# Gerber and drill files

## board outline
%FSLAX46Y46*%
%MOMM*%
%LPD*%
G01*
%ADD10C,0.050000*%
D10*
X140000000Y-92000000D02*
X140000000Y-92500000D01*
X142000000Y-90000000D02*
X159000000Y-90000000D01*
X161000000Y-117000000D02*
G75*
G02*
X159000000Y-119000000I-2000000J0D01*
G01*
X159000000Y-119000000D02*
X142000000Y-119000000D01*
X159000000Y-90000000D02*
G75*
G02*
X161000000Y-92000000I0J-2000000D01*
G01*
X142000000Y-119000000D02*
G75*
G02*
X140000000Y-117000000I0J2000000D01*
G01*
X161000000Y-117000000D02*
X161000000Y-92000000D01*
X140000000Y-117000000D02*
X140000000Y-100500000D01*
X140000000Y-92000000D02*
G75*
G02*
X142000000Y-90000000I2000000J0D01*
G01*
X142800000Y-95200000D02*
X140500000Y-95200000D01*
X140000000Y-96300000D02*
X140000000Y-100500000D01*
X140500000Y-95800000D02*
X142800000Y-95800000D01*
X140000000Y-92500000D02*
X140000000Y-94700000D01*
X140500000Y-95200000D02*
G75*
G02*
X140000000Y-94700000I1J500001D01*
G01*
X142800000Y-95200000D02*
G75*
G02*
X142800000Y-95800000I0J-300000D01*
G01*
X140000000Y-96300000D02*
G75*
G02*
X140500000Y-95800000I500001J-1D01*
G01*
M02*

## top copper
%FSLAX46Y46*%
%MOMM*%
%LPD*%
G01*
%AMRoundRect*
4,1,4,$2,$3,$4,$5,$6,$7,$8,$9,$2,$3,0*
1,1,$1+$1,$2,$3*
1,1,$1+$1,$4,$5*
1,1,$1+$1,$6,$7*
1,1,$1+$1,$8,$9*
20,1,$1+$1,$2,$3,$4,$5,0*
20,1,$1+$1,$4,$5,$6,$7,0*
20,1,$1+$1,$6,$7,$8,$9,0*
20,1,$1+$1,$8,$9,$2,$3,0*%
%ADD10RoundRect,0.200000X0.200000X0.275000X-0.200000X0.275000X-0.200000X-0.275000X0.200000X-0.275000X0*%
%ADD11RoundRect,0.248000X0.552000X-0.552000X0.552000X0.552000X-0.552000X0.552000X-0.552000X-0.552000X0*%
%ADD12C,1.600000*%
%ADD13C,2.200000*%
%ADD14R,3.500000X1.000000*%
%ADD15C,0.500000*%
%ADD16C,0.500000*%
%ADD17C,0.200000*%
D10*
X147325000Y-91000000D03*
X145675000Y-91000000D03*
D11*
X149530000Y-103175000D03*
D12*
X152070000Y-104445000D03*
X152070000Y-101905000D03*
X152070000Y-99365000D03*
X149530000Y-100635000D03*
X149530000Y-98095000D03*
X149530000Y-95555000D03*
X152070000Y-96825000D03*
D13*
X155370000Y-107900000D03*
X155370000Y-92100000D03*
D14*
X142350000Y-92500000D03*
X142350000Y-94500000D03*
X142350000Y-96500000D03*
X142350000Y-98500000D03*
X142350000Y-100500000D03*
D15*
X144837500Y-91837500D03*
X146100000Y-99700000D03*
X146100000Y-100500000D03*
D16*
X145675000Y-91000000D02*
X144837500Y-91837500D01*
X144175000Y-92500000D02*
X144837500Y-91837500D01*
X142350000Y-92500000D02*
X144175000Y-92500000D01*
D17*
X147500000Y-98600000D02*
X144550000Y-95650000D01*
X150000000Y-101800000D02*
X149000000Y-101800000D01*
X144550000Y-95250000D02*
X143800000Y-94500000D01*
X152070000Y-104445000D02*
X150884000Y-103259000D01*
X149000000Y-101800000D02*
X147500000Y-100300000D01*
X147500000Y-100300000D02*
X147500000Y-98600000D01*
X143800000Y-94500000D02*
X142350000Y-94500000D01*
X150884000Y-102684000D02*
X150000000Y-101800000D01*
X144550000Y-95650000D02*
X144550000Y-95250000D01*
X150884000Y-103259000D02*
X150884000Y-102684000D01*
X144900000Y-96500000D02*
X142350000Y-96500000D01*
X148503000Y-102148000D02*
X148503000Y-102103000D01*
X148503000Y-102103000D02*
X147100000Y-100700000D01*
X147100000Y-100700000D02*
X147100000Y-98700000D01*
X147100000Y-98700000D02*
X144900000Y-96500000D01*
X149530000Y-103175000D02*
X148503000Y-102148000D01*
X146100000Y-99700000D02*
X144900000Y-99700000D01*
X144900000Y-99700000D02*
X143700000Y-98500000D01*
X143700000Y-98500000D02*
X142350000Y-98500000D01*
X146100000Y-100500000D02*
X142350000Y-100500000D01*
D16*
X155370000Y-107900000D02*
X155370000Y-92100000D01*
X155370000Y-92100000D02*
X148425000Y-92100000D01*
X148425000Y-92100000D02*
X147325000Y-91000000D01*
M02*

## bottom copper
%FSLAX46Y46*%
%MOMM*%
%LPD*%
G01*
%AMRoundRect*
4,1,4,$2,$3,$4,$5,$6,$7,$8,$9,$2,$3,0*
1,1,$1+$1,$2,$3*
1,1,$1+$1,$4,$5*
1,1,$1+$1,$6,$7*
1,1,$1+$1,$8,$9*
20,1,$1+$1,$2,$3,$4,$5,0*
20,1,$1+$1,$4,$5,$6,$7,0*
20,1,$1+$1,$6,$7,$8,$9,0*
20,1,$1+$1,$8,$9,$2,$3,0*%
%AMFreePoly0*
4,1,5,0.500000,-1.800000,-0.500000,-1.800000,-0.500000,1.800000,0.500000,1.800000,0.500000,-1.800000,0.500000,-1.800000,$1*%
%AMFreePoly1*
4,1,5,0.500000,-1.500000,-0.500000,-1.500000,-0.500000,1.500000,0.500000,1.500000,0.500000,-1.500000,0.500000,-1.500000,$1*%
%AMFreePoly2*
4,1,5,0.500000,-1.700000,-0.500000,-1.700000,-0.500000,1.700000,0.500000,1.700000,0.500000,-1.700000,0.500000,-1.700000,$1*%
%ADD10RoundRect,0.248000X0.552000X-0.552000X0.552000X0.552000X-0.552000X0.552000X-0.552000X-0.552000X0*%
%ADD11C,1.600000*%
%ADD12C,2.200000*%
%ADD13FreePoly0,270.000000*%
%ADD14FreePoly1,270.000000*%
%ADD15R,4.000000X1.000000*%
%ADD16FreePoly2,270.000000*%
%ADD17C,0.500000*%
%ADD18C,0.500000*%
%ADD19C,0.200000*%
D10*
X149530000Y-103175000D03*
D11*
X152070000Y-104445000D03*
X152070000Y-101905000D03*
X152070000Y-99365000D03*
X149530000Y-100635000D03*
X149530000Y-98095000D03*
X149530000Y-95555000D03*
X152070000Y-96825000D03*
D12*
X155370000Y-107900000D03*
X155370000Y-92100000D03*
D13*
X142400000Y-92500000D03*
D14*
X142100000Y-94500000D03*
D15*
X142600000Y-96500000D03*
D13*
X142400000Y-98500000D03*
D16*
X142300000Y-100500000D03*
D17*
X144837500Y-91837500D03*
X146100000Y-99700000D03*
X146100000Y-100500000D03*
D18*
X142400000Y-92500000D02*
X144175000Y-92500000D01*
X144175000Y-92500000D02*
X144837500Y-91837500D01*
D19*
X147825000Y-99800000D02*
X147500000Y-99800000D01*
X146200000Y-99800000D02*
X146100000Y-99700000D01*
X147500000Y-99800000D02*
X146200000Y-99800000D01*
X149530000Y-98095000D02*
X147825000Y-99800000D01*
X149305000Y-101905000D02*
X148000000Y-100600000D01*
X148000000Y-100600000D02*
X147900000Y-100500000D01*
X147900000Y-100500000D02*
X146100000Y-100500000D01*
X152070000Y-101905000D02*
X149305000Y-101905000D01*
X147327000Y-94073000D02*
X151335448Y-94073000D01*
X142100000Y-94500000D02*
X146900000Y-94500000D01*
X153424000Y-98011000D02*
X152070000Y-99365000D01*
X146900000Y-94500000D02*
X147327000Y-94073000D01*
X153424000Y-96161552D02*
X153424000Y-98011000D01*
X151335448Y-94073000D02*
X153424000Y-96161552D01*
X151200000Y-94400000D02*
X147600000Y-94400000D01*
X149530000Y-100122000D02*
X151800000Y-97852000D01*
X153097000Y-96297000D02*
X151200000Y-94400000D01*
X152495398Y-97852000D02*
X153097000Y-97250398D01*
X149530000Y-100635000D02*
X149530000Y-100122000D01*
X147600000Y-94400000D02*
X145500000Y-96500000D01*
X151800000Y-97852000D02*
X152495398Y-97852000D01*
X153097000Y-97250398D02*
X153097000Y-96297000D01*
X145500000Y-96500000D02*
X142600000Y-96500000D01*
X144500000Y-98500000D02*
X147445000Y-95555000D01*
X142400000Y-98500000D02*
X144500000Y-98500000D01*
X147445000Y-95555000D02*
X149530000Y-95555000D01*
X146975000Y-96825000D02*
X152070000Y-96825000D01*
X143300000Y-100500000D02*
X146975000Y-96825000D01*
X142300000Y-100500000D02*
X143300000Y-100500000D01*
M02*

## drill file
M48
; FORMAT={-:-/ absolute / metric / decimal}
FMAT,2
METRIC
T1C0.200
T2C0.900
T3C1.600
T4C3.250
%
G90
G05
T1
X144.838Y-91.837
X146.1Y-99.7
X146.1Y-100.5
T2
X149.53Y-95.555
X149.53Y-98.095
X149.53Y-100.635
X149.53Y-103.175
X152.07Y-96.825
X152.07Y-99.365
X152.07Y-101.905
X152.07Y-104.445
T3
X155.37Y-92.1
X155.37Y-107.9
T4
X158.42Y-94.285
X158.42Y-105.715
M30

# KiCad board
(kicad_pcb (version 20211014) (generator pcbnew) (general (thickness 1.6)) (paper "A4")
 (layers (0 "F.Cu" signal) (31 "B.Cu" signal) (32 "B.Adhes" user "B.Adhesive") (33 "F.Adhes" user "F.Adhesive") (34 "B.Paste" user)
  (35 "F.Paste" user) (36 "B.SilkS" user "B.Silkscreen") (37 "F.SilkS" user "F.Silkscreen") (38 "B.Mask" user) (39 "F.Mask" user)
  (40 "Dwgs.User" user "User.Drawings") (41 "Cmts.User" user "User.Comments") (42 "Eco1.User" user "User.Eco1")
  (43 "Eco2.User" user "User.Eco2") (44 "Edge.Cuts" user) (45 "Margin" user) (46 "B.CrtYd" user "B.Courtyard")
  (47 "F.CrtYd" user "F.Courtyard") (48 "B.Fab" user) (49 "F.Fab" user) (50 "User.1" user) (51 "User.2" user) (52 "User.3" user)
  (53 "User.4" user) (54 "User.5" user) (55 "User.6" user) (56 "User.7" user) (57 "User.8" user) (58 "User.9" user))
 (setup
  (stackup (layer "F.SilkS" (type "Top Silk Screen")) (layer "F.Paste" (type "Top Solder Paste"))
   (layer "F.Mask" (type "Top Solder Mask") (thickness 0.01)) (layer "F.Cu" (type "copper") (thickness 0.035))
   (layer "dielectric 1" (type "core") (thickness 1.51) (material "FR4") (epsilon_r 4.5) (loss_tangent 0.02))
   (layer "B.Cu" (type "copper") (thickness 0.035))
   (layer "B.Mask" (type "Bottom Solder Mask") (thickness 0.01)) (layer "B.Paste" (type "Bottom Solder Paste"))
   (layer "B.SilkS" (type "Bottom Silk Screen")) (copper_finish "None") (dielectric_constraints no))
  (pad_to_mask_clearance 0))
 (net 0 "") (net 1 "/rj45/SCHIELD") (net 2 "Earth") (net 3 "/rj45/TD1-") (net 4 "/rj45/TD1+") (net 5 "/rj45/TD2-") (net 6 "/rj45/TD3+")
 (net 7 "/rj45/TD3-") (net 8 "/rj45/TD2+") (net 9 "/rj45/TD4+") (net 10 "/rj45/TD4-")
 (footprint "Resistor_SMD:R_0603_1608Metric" (layer "F.Cu") (at 146.5 91 180)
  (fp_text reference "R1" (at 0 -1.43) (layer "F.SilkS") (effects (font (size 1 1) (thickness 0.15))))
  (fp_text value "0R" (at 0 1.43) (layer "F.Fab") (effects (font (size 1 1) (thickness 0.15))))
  (pad "1" smd roundrect (at -0.825 0 180) (size 0.8 0.95) (layers "F.Cu" "F.Paste" "F.Mask") (roundrect_rratio 0.25)
   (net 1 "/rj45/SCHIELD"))
  (pad "2" smd roundrect (at 0.825 0 180) (size 0.8 0.95) (layers "F.Cu" "F.Paste" "F.Mask") (roundrect_rratio 0.25) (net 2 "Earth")))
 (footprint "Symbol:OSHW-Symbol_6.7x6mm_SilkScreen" (layer "F.Cu") (at 143.5 115)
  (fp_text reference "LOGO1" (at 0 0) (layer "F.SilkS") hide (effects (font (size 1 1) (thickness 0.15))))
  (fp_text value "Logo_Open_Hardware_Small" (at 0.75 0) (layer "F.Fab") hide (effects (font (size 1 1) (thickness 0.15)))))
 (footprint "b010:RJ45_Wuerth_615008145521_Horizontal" (layer "F.Cu") (at 149.53 95.555)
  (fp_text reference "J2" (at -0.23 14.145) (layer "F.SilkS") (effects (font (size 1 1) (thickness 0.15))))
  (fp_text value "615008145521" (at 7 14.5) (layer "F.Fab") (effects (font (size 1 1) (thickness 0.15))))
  (pad "" np_thru_hole circle (at 8.89 10.16 90) (size 3.25 3.25) (drill 3.25) (layers *.Cu *.Mask))
  (pad "" np_thru_hole circle (at 8.89 -1.27 90) (size 3.25 3.25) (drill 3.25) (layers *.Cu *.Mask))
  (pad "1" thru_hole roundrect (at 0 7.62 90) (size 1.6 1.6) (drill 0.9) (layers *.Cu *.Mask) (roundrect_rratio 0.155) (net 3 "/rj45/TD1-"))
  (pad "2" thru_hole circle (at 2.54 8.89 90) (size 1.6 1.6) (drill 0.9) (layers *.Cu *.Mask) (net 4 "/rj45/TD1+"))
  (pad "3" thru_hole circle (at 2.54 6.35 90) (size 1.6 1.6) (drill 0.9) (layers *.Cu *.Mask) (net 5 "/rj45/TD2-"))
  (pad "4" thru_hole circle (at 2.54 3.81 90) (size 1.6 1.6) (drill 0.9) (layers *.Cu *.Mask) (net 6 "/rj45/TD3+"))
  (pad "5" thru_hole circle (at 0 5.08 90) (size 1.6 1.6) (drill 0.9) (layers *.Cu *.Mask) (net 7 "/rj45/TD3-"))
  (pad "6" thru_hole circle (at 0 2.54 90) (size 1.6 1.6) (drill 0.9) (layers *.Cu *.Mask) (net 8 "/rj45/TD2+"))
  (pad "7" thru_hole circle (at 0 0 90) (size 1.6 1.6) (drill 0.9) (layers *.Cu *.Mask) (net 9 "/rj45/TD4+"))
  (pad "8" thru_hole circle (at 2.54 1.27 90) (size 1.6 1.6) (drill 0.9) (layers *.Cu *.Mask) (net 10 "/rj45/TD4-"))
  (pad "SH" thru_hole circle (at 5.84 12.345 90) (size 2.2 2.2) (drill 1.6) (layers *.Cu *.Mask) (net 1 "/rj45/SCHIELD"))
  (pad "SH" thru_hole circle (at 5.84 -3.455 90) (size 2.2 2.2) (drill 1.6) (layers *.Cu *.Mask) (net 1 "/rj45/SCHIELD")))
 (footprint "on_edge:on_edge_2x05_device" (layer "F.Cu") (at 140 96.5 -90)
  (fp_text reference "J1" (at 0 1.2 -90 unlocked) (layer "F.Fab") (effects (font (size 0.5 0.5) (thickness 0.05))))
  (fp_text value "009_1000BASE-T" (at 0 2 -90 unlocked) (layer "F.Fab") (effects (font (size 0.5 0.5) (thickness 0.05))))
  (fp_line (start -1.3 -2.8) (end -1.3 -0.5) (layer "Edge.Cuts") (width 0.05))
  (fp_line (start -0.2 0) (end 4 0) (layer "Edge.Cuts") (width 0.05))
  (fp_line (start -0.7 -0.5) (end -0.7 -2.8) (layer "Edge.Cuts") (width 0.05))
  (fp_line (start -4 0) (end -1.8 0) (layer "Edge.Cuts") (width 0.05))
  (fp_arc (start -1.3 -0.5) (mid -1.446447 -0.146447) (end -1.8 0) (layer "Edge.Cuts") (width 0.05))
  (fp_arc (start -1.3 -2.8) (mid -1 -3.1) (end -0.7 -2.8) (layer "Edge.Cuts") (width 0.05))
  (fp_arc (start -0.2 0) (mid -0.553553 -0.146447) (end -0.7 -0.5) (layer "Edge.Cuts") (width 0.05))
  (pad "1" smd rect (at -4 -2.35 90) (size 1 3.5) (layers "F.Cu" "F.Mask") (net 2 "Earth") (zone_connect 0))
  (pad "2" smd rect (at -2 -2.35 270) (size 1 3.5) (layers "F.Cu" "F.Mask") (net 4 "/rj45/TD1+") (zone_connect 0))
  (pad "3" smd rect (at 0 -2.35 270) (size 1 3.5) (layers "F.Cu" "F.Mask") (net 3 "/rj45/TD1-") (zone_connect 0))
  (pad "4" smd rect (at 2 -2.35 90) (size 1 3.5) (layers "F.Cu" "F.Mask") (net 8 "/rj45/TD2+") (zone_connect 0))
  (pad "5" smd rect (at 4 -2.35 90) (size 1 3.5) (layers "F.Cu" "F.Mask") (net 5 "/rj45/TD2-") (zone_connect 0))
  (pad "6" smd custom (at -4 -2.4 270) (size 1 3.6) (layers "B.Cu" "B.Mask") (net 2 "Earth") (zone_connect 0)
   (options (clearance outline) (anchor rect)) (primitives))
  (pad "7" smd custom (at -2 -2.1 270) (size 1 3) (layers "B.Cu" "B.Mask") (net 6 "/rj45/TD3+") (zone_connect 0)
   (options (clearance outline) (anchor rect)) (primitives))
  (pad "8" smd rect (at 0 -2.6 270) (size 1 4) (layers "B.Cu" "B.Mask") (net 7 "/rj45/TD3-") (zone_connect 0))
  (pad "9" smd custom (at 2 -2.4 270) (size 1 3.6) (layers "B.Cu" "B.Mask") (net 9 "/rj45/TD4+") (zone_connect 0)
   (options (clearance outline) (anchor rect)) (primitives))
  (pad "10" smd custom (at 4 -2.3 270) (size 1 3.4) (layers "B.Cu" "B.Mask") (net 10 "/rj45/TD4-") (zone_connect 0)
   (options (clearance outline) (anchor rect)) (primitives))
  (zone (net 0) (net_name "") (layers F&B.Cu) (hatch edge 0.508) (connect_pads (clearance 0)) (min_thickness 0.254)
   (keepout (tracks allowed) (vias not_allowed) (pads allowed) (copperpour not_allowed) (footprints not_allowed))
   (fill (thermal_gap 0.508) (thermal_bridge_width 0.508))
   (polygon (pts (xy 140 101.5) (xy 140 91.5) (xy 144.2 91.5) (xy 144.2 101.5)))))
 (gr_line (start 140 92) (end 140 92.5) (layer "Edge.Cuts") (width 0.05))
 (gr_line (start 142 90) (end 159 90) (layer "Edge.Cuts") (width 0.05))
 (gr_arc (start 161 117) (mid 160.414214 118.414214) (end 159 119) (layer "Edge.Cuts") (width 0.05))
 (gr_line (start 159 119) (end 142 119) (layer "Edge.Cuts") (width 0.05))
 (gr_arc (start 159 90) (mid 160.414214 90.585786) (end 161 92) (layer "Edge.Cuts") (width 0.05))
 (gr_arc (start 142 119) (mid 140.585786 118.414214) (end 140 117) (layer "Edge.Cuts") (width 0.05))
 (gr_line (start 161 117) (end 161 92) (layer "Edge.Cuts") (width 0.05))
 (gr_line (start 140 117) (end 140 100.5) (layer "Edge.Cuts") (width 0.05))
 (gr_arc (start 140 92) (mid 140.585786 90.585786) (end 142 90) (layer "Edge.Cuts") (width 0.05))
 (segment (start 145.675 91) (end 144.8375 91.8375) (width 0.5) (layer "F.Cu") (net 2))
 (segment (start 144.175 92.5) (end 144.8375 91.8375) (width 0.5) (layer "F.Cu") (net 2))
 (segment (start 142.35 92.5) (end 144.175 92.5) (width 0.5) (layer "F.Cu") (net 2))
 (via (at 144.8375 91.8375) (size 0.5) (drill 0.2) (layers "F.Cu" "B.Cu") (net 2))
 (segment (start 142.4 92.5) (end 144.175 92.5) (width 0.5) (layer "B.Cu") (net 2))
 (segment (start 144.175 92.5) (end 144.8375 91.8375) (width 0.5) (layer "B.Cu") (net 2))
 (segment (start 147.5 98.6) (end 144.55 95.65) (width 0.2) (layer "F.Cu") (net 4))
 (segment (start 150 101.8) (end 149 101.8) (width 0.2) (layer "F.Cu") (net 4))
 (segment (start 144.55 95.25) (end 143.8 94.5) (width 0.2) (layer "F.Cu") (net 4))
 (segment (start 152.07 104.445) (end 150.884 103.259) (width 0.2) (layer "F.Cu") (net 4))
 (segment (start 149 101.8) (end 147.5 100.3) (width 0.2) (layer "F.Cu") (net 4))
 (segment (start 147.5 100.3) (end 147.5 98.6) (width 0.2) (layer "F.Cu") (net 4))
 (segment (start 143.8 94.5) (end 142.35 94.5) (width 0.2) (layer "F.Cu") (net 4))
 (segment (start 150.884 102.684) (end 150 101.8) (width 0.2) (layer "F.Cu") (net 4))
 (segment (start 144.55 95.65) (end 144.55 95.25) (width 0.2) (layer "F.Cu") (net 4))
 (segment (start 150.884 103.259) (end 150.884 102.684) (width 0.2) (layer "F.Cu") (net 4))
 (segment (start 144.9 96.5) (end 142.35 96.5) (width 0.2) (layer "F.Cu") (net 3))
 (segment (start 148.503 102.148) (end 148.503 102.103) (width 0.2) (layer "F.Cu") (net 3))
 (segment (start 148.503 102.103) (end 147.1 100.7) (width 0.2) (layer "F.Cu") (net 3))
 (segment (start 147.1 100.7) (end 147.1 98.7) (width 0.2) (layer "F.Cu") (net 3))
 (segment (start 147.1 98.7) (end 144.9 96.5) (width 0.2) (layer "F.Cu") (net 3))
 (segment (start 149.53 103.175) (end 148.503 102.148) (width 0.2) (layer "F.Cu") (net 3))
 (segment (start 146.1 99.7) (end 144.9 99.7) (width 0.2) (layer "F.Cu") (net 8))
 (segment (start 144.9 99.7) (end 143.7 98.5) (width 0.2) (layer "F.Cu") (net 8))
 (segment (start 143.7 98.5) (end 142.35 98.5) (width 0.2) (layer "F.Cu") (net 8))
 (via (at 146.1 99.7) (size 0.5) (drill 0.2) (layers "F.Cu" "B.Cu") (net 8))
 (segment (start 147.825 99.8) (end 147.5 99.8) (width 0.2) (layer "B.Cu") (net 8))
 (segment (start 146.2 99.8) (end 146.1 99.7) (width 0.2) (layer "B.Cu") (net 8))
 (segment (start 147.5 99.8) (end 146.2 99.8) (width 0.2) (layer "B.Cu") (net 8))
 (segment (start 149.53 98.095) (end 147.825 99.8) (width 0.2) (layer "B.Cu") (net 8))
 (segment (start 146.1 100.5) (end 142.35 100.5) (width 0.2) (layer "F.Cu") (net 5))
 (via (at 146.1 100.5) (size 0.5) (drill 0.2) (layers "F.Cu" "B.Cu") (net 5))
 (segment (start 149.305 101.905) (end 148 100.6) (width 0.2) (layer "B.Cu") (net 5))
 (segment (start 148 100.6) (end 147.9 100.5) (width 0.2) (layer "B.Cu") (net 5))
 (segment (start 147.9 100.5) (end 146.1 100.5) (width 0.2) (layer "B.Cu") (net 5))
 (segment (start 152.07 101.905) (end 149.305 101.905) (width 0.2) (layer "B.Cu") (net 5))
 (segment (start 147.327 94.073) (end 151.335448 94.073) (width 0.2) (layer "B.Cu") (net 6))
 (segment (start 142.1 94.5) (end 146.9 94.5) (width 0.2) (layer "B.Cu") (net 6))
 (segment (start 153.424 98.011) (end 152.07 99.365) (width 0.2) (layer "B.Cu") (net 6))
 (segment (start 146.9 94.5) (end 147.327 94.073) (width 0.2) (layer "B.Cu") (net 6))
 (segment (start 153.424 96.161552) (end 153.424 98.011) (width 0.2) (layer "B.Cu") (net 6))
 (segment (start 151.335448 94.073) (end 153.424 96.161552) (width 0.2) (layer "B.Cu") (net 6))
 (segment (start 151.2 94.4) (end 147.6 94.4) (width 0.2) (layer "B.Cu") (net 7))
 (segment (start 149.53 100.122) (end 151.8 97.852) (width 0.2) (layer "B.Cu") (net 7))
 (segment (start 153.097 96.297) (end 151.2 94.4) (width 0.2) (layer "B.Cu") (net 7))
 (segment (start 152.495398 97.852) (end 153.097 97.250398) (width 0.2) (layer "B.Cu") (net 7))
 (segment (start 149.53 100.635) (end 149.53 100.122) (width 0.2) (layer "B.Cu") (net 7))
 (segment (start 147.6 94.4) (end 145.5 96.5) (width 0.2) (layer "B.Cu") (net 7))
 (segment (start 151.8 97.852) (end 152.495398 97.852) (width 0.2) (layer "B.Cu") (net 7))
 (segment (start 153.097 97.250398) (end 153.097 96.297) (width 0.2) (layer "B.Cu") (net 7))
 (segment (start 145.5 96.5) (end 142.6 96.5) (width 0.2) (layer "B.Cu") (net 7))
 (segment (start 144.5 98.5) (end 147.445 95.555) (width 0.2) (layer "B.Cu") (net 9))
 (segment (start 142.4 98.5) (end 144.5 98.5) (width 0.2) (layer "B.Cu") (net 9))
 (segment (start 147.445 95.555) (end 149.53 95.555) (width 0.2) (layer "B.Cu") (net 9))
 (segment (start 146.975 96.825) (end 152.07 96.825) (width 0.2) (layer "B.Cu") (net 10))
 (segment (start 143.3 100.5) (end 146.975 96.825) (width 0.2) (layer "B.Cu") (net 10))
 (segment (start 142.3 100.5) (end 143.3 100.5) (width 0.2) (layer "B.Cu") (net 10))
 (segment (start 155.37 107.9) (end 155.37 92.1) (width 0.5) (layer "F.Cu") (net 1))
 (segment (start 155.37 92.1) (end 148.425 92.1) (width 0.5) (layer "F.Cu") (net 1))
 (segment (start 148.425 92.1) (end 147.325 91) (width 0.5) (layer "F.Cu") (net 1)))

